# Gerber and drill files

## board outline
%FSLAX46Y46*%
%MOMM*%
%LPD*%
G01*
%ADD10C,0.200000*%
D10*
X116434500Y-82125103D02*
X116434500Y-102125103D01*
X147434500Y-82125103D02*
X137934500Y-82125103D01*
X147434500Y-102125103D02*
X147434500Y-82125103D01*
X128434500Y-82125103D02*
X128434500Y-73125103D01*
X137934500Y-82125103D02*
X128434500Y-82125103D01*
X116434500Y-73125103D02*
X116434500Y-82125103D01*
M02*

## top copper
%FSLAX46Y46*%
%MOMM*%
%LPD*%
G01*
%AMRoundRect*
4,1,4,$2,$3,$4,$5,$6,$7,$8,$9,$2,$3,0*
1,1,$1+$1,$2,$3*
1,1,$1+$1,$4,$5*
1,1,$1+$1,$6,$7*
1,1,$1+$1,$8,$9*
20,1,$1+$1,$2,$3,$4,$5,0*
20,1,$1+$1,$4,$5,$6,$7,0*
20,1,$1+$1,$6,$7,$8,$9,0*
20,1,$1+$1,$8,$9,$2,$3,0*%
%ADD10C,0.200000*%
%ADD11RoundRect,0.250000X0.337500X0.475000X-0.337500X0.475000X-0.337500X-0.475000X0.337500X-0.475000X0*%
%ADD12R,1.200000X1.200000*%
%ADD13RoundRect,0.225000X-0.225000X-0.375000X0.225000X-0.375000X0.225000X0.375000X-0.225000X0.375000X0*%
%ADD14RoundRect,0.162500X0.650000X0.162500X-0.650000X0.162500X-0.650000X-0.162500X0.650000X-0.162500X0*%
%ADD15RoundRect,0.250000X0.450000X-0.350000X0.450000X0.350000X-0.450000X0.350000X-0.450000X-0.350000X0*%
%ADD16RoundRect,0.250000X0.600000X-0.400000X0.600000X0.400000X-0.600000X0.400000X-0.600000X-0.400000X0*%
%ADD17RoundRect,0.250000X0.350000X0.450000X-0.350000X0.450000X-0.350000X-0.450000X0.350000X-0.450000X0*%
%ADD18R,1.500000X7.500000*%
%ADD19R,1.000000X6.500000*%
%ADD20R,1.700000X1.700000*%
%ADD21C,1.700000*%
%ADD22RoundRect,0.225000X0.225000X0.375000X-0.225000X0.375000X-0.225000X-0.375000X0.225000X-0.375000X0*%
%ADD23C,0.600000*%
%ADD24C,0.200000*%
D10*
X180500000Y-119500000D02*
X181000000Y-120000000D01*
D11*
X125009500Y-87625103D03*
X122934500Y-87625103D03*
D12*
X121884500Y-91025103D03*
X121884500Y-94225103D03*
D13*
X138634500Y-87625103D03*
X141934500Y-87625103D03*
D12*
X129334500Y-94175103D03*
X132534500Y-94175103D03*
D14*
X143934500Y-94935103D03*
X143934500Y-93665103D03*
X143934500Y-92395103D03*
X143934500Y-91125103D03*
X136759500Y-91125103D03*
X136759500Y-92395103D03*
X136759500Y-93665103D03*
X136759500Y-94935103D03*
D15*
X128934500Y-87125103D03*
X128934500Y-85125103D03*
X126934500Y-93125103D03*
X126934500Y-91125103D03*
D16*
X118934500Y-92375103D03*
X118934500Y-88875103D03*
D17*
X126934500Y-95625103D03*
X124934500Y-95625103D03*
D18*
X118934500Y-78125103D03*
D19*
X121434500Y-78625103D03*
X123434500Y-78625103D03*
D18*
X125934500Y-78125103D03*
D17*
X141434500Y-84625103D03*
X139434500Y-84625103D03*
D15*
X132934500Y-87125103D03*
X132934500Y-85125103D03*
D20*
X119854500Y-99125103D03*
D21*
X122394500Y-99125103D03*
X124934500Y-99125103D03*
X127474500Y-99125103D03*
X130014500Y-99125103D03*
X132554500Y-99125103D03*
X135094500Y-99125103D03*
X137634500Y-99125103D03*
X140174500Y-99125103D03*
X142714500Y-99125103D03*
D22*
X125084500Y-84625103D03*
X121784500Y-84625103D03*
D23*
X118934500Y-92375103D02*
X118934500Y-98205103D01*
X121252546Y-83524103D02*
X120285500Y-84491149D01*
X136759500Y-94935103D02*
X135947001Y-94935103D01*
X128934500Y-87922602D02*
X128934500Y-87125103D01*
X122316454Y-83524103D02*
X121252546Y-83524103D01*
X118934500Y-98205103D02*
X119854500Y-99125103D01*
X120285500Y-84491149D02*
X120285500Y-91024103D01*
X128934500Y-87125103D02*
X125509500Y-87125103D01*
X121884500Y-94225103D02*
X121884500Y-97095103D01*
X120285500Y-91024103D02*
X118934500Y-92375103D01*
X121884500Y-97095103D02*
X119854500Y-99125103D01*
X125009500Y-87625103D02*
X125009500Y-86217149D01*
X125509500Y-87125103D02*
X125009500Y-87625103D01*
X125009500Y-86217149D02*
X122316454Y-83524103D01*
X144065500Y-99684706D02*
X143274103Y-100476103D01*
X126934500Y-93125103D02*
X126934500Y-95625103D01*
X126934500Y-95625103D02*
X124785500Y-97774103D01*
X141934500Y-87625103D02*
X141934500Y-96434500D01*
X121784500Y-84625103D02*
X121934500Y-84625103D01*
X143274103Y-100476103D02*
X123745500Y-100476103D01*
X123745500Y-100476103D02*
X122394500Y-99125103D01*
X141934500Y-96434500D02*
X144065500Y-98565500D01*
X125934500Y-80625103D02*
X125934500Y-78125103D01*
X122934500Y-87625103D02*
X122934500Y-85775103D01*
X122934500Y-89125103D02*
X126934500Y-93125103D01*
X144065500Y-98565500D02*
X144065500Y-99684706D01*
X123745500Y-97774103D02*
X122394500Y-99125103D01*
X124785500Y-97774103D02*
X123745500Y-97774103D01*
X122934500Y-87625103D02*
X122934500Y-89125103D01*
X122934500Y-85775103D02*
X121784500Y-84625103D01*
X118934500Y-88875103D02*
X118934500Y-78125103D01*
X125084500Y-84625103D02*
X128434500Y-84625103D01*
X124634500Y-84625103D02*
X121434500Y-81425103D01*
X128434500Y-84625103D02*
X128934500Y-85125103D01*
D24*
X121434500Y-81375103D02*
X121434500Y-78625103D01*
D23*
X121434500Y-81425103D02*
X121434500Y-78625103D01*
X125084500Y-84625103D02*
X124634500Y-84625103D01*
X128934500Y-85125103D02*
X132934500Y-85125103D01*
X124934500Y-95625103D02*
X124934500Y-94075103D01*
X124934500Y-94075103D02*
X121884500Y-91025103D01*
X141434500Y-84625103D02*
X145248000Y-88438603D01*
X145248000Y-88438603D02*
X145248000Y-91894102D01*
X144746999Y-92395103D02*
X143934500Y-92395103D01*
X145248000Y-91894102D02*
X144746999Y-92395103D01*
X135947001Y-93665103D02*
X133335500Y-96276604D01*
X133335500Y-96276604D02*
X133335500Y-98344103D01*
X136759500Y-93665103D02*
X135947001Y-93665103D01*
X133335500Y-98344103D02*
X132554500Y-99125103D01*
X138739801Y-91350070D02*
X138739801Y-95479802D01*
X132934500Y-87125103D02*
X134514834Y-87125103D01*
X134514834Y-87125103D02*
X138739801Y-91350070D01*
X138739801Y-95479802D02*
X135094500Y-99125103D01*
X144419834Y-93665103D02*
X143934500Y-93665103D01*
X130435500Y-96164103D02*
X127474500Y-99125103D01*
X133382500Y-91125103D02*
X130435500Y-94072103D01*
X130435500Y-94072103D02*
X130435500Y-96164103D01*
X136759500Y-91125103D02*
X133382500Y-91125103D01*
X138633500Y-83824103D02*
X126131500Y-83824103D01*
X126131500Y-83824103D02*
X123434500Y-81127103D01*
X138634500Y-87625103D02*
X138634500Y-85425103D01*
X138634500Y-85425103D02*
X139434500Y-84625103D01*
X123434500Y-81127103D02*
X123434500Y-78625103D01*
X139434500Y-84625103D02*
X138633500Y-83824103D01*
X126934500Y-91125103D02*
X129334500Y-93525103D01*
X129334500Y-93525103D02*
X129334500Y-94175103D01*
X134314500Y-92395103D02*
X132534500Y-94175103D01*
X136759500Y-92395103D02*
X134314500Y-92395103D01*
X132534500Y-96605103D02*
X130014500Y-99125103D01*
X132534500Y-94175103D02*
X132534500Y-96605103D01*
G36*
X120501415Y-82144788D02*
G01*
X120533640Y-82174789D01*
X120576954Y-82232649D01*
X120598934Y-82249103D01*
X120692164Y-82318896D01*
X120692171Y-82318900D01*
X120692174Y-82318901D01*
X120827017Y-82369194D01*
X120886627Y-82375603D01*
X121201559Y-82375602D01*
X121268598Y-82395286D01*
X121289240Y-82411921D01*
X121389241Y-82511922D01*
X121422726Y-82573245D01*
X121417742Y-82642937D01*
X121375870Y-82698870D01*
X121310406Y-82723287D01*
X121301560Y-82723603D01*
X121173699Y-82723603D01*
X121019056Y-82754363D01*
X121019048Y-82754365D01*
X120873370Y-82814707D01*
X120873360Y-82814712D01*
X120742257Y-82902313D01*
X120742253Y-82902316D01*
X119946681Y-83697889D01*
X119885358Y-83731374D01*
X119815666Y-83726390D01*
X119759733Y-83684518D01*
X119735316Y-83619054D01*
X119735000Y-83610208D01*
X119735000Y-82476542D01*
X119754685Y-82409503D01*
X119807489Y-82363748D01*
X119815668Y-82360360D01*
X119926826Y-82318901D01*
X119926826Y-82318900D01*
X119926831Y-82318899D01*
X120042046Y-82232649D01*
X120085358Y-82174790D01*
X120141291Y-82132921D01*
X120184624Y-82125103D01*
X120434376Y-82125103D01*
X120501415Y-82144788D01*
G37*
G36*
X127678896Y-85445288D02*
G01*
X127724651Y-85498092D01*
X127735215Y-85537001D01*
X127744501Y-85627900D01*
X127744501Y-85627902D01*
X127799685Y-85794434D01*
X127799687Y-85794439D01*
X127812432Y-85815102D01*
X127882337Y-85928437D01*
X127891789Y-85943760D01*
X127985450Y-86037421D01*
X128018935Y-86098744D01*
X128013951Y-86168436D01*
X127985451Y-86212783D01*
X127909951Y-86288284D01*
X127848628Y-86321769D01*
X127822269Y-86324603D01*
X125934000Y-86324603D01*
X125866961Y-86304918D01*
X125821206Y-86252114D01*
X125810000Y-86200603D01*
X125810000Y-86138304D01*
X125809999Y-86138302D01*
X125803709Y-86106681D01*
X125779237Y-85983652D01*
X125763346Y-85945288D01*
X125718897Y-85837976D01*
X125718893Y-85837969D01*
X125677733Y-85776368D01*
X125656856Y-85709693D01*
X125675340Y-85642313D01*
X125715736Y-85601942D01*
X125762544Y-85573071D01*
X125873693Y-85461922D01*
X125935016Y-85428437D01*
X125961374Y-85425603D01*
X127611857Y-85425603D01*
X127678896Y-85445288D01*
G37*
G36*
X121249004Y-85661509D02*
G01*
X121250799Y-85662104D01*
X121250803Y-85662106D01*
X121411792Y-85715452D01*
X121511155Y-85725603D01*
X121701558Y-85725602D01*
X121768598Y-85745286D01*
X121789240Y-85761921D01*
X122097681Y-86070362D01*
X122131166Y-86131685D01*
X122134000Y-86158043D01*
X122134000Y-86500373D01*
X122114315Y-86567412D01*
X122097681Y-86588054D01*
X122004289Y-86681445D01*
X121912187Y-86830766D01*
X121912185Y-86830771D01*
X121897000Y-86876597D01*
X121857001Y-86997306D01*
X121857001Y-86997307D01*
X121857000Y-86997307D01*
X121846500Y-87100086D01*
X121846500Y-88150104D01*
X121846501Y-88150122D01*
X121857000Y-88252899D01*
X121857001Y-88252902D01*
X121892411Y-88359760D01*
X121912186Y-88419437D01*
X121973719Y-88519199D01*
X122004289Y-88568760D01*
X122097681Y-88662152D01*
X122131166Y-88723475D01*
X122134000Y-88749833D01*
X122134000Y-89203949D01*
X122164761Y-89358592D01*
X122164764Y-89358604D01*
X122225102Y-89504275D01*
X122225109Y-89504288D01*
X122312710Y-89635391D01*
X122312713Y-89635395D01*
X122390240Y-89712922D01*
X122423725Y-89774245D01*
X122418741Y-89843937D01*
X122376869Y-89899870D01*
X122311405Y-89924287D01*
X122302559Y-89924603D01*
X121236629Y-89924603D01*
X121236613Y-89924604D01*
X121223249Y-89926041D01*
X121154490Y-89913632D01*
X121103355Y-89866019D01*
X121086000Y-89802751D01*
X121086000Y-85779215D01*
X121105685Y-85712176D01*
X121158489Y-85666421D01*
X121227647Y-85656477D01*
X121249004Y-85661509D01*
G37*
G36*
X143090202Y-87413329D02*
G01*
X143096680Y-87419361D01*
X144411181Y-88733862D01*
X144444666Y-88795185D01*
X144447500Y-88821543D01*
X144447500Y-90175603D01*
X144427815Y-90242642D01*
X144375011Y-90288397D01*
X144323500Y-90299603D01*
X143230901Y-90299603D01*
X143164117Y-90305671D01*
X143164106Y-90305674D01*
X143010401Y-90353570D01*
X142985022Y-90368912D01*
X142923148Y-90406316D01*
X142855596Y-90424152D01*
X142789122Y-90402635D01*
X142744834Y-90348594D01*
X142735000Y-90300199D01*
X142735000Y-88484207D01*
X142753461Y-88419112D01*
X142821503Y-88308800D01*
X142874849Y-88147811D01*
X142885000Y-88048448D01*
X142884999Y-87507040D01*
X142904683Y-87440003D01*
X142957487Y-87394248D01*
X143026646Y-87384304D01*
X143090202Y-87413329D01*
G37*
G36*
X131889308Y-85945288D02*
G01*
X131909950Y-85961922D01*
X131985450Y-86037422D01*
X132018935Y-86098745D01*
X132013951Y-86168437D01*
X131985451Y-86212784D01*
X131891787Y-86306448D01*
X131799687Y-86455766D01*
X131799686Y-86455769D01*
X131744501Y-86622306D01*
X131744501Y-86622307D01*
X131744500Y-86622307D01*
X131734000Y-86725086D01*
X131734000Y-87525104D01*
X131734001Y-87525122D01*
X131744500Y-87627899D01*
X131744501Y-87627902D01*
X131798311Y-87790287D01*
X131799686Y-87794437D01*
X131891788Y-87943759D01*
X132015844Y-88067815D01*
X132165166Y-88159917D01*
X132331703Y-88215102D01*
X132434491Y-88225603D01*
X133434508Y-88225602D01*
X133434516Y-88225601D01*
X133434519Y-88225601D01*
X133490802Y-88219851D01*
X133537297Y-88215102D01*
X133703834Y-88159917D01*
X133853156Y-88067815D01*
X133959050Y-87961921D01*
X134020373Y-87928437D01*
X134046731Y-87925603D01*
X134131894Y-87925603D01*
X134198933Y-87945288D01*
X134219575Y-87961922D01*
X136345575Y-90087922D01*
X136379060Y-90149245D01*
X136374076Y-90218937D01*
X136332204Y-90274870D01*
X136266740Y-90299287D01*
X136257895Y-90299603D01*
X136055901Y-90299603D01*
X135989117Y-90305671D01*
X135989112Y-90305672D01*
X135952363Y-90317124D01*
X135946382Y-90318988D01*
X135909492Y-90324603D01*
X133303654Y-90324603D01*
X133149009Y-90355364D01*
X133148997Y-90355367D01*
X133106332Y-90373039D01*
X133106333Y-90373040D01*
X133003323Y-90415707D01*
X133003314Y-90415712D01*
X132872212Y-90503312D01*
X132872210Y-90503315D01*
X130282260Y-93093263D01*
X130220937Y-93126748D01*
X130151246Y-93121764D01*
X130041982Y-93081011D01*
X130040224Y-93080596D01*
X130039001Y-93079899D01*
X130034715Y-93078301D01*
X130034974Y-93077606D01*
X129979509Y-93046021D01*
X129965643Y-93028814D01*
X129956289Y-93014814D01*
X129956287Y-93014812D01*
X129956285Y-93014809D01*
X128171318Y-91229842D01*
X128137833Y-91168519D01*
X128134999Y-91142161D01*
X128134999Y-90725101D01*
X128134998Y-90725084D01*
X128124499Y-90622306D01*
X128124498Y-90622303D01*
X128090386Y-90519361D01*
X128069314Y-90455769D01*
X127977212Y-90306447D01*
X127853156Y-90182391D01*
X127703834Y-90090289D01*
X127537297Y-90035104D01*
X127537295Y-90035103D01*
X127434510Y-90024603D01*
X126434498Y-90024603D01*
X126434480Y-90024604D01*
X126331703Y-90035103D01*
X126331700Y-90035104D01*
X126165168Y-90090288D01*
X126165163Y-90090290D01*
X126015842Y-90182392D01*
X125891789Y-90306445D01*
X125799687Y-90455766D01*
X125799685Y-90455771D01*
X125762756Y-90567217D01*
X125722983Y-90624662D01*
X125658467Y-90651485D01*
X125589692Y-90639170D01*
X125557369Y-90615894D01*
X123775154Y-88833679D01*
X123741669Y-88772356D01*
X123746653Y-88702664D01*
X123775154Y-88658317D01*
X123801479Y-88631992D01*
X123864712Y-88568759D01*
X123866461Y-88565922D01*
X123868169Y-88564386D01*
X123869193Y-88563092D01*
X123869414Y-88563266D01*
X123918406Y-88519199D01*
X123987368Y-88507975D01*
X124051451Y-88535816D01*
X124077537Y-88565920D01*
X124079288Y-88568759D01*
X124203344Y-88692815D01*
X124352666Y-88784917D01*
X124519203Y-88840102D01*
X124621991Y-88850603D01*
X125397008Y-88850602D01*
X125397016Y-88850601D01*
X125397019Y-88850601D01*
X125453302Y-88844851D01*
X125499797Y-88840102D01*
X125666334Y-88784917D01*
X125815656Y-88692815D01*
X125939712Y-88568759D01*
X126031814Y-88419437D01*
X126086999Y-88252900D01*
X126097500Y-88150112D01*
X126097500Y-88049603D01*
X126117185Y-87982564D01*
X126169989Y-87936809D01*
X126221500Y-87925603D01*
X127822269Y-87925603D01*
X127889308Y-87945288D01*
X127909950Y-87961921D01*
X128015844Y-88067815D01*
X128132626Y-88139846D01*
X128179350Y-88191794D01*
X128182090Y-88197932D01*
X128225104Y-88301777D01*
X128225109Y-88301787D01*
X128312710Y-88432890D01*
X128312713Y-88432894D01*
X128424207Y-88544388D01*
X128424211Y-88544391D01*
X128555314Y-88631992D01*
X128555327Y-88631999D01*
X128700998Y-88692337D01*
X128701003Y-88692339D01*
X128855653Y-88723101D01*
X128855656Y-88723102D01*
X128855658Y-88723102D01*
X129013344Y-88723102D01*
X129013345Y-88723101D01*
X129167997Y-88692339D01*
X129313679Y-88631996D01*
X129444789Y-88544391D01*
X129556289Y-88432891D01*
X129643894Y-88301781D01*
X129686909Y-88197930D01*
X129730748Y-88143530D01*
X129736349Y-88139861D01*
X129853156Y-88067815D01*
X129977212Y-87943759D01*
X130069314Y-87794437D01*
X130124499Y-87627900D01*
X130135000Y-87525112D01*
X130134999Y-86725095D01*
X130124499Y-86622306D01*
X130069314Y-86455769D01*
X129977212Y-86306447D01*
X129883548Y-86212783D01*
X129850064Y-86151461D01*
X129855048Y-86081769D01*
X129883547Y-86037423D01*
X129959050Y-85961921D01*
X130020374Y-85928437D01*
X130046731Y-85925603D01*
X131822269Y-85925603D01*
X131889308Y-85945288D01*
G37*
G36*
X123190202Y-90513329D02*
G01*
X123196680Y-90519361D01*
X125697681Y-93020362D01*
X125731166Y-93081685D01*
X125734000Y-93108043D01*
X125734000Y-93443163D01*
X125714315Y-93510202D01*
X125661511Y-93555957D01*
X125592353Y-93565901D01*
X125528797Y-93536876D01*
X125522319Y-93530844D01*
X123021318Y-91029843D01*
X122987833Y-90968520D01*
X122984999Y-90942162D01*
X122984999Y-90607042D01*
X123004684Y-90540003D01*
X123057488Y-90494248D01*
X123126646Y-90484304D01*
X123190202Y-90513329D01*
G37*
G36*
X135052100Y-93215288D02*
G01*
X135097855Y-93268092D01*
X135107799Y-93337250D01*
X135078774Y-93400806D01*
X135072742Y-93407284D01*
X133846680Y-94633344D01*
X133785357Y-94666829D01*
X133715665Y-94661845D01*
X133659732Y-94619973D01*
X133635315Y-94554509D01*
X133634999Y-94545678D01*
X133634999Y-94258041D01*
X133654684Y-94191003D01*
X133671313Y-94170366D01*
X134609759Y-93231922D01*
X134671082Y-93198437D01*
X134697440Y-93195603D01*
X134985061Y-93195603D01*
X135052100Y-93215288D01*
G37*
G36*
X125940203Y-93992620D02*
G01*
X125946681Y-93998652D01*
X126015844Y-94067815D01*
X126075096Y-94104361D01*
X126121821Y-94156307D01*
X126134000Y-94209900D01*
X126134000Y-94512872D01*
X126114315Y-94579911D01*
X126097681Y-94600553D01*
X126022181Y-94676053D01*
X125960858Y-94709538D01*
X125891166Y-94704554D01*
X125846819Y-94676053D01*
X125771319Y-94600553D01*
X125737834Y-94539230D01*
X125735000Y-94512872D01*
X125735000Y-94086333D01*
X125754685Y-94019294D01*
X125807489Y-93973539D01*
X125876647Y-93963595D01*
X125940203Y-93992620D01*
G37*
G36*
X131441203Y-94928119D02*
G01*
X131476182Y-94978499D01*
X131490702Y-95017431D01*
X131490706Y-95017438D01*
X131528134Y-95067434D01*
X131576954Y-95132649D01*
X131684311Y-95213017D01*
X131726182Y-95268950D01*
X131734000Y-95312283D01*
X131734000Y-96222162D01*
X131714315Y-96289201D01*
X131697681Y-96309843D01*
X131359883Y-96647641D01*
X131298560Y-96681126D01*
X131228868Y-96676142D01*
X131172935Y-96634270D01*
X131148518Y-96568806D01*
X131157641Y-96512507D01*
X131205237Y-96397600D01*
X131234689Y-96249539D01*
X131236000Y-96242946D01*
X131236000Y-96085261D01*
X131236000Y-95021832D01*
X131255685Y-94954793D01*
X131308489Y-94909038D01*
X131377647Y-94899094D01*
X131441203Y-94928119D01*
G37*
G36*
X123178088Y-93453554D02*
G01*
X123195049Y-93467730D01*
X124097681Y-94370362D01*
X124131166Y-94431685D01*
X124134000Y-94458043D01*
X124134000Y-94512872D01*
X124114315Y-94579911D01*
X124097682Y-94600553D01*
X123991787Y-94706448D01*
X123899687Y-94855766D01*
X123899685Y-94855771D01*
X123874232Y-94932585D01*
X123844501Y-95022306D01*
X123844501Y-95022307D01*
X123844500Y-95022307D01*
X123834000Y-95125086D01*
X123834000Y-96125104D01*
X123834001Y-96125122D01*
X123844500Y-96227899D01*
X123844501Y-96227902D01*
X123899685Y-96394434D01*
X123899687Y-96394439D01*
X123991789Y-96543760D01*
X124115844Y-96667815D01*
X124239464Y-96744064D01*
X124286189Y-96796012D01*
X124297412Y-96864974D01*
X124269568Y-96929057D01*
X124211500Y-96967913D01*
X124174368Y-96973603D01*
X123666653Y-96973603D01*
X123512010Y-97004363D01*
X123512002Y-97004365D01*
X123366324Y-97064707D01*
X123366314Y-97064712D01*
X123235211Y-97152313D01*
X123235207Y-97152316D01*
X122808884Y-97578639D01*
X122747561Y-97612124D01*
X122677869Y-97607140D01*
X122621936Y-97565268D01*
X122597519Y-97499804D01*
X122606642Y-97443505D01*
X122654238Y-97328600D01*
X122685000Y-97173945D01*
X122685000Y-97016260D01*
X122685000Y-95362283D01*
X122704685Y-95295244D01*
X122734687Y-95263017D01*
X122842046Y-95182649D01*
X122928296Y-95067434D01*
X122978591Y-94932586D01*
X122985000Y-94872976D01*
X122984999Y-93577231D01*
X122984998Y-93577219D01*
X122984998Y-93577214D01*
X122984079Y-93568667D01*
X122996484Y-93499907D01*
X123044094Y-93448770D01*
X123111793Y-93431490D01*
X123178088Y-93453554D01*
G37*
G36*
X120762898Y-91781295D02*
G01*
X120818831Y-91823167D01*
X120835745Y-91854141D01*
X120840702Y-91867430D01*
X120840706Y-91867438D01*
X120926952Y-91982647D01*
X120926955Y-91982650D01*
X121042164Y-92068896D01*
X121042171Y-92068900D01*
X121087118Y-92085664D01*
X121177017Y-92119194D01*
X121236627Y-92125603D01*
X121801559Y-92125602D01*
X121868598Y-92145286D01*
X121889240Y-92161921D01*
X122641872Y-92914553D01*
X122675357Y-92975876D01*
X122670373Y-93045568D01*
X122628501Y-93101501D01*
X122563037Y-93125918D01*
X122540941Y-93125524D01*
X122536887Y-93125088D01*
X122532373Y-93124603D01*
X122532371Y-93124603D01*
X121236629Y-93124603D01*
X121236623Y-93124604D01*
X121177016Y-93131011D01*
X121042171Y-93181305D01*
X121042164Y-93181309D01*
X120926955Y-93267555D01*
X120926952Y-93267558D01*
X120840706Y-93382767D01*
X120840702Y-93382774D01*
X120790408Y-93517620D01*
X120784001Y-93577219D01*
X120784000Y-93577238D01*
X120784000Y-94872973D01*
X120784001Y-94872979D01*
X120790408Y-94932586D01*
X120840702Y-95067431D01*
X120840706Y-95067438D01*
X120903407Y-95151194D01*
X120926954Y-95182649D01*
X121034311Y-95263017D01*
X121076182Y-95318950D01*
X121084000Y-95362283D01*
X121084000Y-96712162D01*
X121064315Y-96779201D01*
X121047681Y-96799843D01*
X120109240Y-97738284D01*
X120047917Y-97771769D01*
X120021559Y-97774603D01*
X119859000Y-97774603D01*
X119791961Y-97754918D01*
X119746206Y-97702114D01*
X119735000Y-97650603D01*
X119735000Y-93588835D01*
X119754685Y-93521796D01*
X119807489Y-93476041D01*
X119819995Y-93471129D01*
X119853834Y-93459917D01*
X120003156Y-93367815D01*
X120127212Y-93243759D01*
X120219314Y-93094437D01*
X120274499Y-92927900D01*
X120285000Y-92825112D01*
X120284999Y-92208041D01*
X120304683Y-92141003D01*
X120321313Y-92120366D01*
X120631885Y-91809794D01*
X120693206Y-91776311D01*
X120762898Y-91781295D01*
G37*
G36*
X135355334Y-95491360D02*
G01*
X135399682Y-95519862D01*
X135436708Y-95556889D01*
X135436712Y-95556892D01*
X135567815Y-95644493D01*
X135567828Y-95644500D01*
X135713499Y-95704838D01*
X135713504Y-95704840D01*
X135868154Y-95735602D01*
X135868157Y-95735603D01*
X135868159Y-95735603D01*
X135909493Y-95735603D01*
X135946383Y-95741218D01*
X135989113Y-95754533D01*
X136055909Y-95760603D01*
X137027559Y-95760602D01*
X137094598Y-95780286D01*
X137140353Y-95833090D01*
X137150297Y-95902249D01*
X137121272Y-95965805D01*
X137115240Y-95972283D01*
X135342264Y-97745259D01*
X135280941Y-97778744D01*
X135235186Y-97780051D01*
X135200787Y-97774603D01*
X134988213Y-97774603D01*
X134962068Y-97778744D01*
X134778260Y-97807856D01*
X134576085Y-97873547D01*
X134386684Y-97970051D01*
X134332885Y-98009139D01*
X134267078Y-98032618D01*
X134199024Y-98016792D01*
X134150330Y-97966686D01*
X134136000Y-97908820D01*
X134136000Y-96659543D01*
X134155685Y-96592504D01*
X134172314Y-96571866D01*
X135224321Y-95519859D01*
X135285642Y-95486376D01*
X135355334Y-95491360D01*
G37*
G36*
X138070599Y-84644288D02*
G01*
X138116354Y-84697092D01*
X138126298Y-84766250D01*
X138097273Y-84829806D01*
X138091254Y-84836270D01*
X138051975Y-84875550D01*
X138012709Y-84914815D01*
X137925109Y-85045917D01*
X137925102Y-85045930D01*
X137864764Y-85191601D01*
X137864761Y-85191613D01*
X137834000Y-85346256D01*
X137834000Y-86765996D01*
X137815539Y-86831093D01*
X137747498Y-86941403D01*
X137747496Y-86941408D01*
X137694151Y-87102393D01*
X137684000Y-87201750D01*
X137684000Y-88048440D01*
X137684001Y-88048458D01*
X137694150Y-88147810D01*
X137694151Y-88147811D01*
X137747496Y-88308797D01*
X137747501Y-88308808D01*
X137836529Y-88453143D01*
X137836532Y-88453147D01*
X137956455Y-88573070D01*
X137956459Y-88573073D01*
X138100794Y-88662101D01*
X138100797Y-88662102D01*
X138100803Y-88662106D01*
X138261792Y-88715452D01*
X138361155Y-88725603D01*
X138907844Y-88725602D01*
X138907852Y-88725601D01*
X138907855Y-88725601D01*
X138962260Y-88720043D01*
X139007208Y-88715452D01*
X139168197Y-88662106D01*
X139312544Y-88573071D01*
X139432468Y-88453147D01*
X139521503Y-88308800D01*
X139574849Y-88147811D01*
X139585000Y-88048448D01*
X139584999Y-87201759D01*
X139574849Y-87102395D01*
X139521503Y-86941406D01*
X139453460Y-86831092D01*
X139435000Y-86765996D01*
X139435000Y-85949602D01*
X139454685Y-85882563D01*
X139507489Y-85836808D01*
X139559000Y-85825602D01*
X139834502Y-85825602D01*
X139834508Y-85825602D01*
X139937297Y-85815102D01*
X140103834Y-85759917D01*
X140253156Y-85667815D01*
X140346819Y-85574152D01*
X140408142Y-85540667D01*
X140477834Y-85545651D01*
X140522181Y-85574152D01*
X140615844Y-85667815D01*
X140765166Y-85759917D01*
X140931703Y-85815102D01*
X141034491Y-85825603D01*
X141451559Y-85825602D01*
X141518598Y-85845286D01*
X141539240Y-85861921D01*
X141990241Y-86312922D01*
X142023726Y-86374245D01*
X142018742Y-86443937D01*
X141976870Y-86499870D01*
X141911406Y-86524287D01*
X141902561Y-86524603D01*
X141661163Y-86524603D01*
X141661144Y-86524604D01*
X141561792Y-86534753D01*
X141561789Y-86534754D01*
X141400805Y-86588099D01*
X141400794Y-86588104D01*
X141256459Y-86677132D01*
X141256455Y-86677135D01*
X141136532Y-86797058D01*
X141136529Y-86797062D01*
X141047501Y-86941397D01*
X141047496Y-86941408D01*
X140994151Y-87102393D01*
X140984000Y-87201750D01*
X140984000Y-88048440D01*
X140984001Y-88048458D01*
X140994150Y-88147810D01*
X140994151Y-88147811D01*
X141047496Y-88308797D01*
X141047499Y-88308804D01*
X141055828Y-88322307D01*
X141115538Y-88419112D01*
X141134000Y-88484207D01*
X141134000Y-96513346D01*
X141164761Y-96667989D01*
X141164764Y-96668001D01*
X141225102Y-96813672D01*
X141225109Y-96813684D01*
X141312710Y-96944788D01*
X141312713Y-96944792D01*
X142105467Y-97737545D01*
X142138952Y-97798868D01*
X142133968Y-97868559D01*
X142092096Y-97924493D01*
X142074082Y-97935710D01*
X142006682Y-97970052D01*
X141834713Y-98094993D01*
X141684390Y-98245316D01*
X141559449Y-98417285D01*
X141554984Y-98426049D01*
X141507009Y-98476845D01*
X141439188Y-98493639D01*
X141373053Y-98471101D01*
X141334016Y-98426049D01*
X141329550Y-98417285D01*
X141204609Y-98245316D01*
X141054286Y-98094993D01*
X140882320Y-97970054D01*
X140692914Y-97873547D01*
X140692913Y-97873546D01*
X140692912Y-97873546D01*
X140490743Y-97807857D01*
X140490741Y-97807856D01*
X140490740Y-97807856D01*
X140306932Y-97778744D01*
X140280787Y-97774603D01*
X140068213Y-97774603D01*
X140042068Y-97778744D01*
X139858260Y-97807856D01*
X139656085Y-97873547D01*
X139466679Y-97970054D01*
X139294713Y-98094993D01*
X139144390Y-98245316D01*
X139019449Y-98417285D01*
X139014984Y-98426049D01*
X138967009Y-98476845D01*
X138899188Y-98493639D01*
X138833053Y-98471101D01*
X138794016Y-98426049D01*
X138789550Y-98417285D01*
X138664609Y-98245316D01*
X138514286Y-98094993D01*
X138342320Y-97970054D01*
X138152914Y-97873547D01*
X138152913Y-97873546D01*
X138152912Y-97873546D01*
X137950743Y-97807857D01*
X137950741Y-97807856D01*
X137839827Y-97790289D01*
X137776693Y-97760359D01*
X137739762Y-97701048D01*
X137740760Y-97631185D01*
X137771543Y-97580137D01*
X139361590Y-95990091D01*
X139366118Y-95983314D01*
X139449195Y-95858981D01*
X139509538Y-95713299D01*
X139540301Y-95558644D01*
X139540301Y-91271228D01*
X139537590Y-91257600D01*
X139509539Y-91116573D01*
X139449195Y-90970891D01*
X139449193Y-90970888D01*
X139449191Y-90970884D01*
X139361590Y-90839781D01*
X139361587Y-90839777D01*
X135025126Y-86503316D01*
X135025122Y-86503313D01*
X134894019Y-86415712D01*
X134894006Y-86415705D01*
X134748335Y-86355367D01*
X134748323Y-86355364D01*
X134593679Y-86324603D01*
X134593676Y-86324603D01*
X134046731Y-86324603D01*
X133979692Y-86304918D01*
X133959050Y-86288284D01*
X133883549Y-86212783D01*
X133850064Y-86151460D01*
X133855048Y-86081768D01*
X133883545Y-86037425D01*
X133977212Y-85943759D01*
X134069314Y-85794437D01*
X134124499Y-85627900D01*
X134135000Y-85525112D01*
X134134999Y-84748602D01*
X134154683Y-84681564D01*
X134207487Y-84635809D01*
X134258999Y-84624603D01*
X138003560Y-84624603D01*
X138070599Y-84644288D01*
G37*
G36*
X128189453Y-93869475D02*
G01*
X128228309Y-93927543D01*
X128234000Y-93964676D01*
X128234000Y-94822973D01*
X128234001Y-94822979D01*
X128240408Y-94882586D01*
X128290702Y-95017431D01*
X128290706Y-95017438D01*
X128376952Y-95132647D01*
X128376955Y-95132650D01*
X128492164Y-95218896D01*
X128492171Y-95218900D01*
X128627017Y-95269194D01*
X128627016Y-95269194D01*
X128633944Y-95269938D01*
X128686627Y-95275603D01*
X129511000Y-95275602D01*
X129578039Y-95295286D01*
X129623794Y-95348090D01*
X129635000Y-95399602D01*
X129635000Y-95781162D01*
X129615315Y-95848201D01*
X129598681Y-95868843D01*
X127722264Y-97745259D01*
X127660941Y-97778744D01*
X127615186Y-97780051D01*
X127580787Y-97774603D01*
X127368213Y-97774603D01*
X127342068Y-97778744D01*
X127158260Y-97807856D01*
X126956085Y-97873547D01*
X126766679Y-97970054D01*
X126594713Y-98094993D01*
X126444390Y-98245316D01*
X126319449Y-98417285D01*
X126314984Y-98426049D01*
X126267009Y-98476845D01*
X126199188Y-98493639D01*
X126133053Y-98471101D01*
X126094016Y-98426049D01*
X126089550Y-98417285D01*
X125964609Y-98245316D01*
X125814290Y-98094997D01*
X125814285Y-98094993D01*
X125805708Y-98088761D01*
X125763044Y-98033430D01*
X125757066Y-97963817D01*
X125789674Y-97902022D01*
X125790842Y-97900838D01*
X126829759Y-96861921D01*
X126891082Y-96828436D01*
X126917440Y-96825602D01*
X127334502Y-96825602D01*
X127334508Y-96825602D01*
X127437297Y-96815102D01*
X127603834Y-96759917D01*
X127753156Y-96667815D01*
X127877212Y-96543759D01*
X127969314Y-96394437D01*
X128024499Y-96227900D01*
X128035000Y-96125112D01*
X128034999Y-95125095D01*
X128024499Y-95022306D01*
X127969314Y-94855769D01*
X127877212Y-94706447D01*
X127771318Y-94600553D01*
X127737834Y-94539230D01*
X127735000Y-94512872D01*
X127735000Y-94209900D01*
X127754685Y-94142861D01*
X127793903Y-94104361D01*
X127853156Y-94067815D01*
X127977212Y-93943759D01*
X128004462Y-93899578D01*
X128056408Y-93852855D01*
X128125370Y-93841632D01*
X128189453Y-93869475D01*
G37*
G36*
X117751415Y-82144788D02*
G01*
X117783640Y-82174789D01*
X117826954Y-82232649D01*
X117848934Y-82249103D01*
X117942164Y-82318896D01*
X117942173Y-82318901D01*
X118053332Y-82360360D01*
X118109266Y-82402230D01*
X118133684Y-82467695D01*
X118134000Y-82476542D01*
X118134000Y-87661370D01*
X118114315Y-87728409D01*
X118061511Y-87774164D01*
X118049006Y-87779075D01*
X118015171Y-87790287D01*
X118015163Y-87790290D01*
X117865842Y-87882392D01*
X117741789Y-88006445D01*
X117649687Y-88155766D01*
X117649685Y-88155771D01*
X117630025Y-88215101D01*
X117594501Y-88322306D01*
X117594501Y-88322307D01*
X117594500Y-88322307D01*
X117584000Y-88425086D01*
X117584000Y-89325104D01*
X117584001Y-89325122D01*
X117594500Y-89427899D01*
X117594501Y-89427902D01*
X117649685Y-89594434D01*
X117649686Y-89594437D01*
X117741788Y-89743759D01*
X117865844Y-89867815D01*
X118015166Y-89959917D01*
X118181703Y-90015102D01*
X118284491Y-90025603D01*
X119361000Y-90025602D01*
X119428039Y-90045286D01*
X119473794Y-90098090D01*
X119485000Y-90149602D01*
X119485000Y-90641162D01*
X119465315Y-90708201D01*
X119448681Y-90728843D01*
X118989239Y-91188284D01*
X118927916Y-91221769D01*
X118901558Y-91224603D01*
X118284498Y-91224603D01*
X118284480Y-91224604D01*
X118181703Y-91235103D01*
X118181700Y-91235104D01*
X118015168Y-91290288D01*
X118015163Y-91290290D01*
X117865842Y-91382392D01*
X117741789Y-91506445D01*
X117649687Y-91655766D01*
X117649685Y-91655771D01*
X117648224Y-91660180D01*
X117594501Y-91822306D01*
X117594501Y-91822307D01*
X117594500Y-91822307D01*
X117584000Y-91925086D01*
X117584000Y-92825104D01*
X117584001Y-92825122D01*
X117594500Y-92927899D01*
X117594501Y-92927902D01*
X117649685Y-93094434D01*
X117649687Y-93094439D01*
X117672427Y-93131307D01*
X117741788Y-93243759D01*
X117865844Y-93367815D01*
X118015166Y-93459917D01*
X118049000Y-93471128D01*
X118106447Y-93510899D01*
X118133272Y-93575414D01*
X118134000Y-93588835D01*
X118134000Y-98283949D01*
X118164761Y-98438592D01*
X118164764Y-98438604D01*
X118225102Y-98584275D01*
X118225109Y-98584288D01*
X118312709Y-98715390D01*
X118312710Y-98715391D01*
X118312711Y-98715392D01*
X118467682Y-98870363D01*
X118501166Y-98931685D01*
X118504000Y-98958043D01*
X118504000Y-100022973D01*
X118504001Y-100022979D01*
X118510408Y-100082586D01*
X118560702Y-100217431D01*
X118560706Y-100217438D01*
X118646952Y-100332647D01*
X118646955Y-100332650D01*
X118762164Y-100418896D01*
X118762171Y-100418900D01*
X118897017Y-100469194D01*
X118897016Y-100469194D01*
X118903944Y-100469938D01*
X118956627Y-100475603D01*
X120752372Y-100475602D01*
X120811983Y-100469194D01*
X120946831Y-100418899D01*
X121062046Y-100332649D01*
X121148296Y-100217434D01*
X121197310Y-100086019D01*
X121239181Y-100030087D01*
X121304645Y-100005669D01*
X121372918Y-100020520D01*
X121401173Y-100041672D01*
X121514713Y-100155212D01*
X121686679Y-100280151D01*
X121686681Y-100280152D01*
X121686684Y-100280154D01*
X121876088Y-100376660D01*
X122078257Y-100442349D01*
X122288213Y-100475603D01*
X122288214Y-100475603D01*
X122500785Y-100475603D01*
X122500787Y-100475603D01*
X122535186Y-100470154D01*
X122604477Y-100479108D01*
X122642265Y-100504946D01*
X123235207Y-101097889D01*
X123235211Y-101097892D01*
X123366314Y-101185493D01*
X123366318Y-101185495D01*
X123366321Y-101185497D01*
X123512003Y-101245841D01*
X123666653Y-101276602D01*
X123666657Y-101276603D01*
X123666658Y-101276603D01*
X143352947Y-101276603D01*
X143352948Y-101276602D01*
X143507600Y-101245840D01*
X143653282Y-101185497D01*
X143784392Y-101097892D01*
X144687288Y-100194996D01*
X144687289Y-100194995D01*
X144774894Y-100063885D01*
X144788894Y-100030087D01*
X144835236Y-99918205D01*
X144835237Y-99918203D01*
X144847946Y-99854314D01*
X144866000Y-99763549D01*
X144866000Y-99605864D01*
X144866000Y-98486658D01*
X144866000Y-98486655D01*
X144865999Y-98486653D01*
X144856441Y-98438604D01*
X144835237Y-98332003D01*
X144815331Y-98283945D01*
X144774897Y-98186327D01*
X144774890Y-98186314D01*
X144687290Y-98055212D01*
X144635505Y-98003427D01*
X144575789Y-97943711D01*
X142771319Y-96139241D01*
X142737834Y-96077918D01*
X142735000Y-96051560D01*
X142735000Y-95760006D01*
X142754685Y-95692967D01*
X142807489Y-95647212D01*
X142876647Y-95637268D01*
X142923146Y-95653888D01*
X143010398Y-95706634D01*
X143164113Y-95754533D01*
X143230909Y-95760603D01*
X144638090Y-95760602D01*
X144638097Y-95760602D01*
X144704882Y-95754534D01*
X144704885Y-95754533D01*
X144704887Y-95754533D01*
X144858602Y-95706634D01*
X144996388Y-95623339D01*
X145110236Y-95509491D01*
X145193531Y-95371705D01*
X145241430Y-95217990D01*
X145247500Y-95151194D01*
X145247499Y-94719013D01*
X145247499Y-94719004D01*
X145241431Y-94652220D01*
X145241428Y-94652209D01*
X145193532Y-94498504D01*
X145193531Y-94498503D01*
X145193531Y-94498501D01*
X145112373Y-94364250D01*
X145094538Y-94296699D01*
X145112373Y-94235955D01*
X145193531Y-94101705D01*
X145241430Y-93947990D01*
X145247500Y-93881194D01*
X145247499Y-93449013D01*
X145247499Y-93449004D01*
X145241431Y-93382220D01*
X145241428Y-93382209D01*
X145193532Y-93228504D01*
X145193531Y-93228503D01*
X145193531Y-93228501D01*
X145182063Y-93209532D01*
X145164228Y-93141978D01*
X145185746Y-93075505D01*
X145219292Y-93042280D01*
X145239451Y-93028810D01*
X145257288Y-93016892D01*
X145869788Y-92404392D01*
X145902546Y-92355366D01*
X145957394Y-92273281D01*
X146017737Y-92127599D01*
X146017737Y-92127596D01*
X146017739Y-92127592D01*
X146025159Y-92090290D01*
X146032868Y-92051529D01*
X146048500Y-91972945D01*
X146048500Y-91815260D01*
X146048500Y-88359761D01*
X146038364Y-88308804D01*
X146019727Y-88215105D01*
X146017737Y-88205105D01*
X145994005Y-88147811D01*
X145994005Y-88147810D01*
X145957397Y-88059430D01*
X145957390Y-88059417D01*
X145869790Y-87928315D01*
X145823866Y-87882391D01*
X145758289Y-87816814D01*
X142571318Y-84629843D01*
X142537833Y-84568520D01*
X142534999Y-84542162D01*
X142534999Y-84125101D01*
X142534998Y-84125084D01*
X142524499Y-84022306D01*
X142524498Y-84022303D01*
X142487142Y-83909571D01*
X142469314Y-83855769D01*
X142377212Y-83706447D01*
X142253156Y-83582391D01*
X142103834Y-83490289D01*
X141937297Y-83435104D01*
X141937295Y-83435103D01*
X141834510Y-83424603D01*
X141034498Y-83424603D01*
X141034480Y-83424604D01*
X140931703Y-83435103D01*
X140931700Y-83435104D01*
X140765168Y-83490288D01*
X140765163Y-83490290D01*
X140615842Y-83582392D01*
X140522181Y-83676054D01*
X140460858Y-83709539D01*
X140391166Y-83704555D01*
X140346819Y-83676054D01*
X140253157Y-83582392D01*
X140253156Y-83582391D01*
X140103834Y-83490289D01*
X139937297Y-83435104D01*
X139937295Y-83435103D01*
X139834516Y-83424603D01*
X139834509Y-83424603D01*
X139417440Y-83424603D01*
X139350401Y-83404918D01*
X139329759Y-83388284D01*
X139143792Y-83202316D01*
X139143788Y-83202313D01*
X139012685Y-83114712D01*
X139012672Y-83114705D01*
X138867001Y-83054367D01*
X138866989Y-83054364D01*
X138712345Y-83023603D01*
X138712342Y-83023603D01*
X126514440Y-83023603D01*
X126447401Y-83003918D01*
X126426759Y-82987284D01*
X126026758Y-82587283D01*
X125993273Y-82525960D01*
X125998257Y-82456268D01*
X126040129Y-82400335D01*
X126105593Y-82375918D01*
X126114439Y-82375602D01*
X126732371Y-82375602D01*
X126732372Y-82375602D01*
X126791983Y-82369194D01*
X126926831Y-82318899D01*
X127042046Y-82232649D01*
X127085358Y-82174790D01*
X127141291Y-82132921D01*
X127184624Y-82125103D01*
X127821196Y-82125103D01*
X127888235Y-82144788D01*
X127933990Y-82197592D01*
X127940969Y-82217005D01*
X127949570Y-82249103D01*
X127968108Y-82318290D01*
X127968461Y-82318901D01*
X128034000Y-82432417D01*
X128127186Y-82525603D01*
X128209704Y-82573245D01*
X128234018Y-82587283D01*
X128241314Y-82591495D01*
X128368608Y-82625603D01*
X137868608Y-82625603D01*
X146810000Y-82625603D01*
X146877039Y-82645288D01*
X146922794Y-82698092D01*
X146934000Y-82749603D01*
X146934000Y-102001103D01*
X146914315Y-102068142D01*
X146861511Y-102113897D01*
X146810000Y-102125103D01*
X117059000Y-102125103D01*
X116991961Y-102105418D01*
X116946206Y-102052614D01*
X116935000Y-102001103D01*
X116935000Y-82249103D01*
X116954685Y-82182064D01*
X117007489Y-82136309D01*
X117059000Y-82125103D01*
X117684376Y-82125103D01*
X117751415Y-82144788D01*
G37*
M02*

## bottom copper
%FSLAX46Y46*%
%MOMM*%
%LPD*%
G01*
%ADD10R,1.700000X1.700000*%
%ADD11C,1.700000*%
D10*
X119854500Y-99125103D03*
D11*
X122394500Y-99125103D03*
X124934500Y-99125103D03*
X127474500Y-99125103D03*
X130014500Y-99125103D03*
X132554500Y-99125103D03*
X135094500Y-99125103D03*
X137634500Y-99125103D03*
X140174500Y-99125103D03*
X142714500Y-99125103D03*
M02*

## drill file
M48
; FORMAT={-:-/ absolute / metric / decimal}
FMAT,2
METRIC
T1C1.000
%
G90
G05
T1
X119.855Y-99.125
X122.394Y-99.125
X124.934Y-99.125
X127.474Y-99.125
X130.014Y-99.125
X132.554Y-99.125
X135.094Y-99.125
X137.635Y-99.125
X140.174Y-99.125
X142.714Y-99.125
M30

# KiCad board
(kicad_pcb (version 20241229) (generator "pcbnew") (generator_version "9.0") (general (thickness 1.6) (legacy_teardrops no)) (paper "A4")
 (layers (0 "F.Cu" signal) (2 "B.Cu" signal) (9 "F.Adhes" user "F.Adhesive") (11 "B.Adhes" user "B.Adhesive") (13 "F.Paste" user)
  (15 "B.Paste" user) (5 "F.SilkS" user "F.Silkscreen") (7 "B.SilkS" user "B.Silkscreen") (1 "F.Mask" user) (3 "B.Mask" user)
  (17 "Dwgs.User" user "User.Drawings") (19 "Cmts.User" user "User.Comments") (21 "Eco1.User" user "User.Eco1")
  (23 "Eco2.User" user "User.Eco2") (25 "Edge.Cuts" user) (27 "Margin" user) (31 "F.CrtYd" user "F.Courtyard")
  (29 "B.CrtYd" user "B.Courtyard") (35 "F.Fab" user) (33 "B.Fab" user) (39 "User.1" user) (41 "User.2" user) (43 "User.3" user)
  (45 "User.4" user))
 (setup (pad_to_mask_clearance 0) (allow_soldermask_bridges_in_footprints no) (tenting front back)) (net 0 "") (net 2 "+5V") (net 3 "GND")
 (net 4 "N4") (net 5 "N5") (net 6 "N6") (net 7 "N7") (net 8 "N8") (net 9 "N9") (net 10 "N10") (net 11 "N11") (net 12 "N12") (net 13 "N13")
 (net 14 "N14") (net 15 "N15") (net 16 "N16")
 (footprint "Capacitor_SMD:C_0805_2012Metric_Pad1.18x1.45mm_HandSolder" (layer "F.Cu") (at 123.972 87.625103 180)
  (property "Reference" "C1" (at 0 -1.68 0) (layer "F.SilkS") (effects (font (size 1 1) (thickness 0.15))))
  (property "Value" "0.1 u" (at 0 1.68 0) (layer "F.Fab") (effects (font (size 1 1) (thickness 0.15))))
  (pad "1" smd roundrect (at -1.0375 0 180) (size 1.175 1.45) (layers "F.Cu" "F.Mask" "F.Paste") (roundrect_rratio 0.212766) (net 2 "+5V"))
  (pad "2" smd roundrect (at 1.0375 0 180) (size 1.175 1.45) (layers "F.Cu" "F.Mask" "F.Paste") (roundrect_rratio 0.212766) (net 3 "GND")))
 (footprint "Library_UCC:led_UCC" (layer "F.Cu") (at 122.3345 93.125103 -90)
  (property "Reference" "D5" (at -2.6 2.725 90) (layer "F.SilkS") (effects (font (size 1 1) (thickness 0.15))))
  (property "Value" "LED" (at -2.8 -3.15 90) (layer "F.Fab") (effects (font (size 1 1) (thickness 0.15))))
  (pad "1" smd rect (at -2.1 0.45 270) (size 1.2 1.2) (layers "F.Cu" "F.Mask" "F.Paste") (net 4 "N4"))
  (pad "2" smd rect (at 1.1 0.45 270) (size 1.2 1.2) (layers "F.Cu" "F.Mask" "F.Paste") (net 2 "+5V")))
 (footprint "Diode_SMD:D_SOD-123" (layer "F.Cu") (at 140.2845 87.625103)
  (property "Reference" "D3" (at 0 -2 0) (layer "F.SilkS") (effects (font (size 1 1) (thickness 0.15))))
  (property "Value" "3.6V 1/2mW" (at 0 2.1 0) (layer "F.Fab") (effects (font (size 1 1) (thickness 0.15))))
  (pad "1" smd roundrect (at -1.65 0) (size 0.9 1.2) (layers "F.Cu" "F.Mask" "F.Paste") (roundrect_rratio 0.25) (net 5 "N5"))
  (pad "2" smd roundrect (at 1.65 0) (size 0.9 1.2) (layers "F.Cu" "F.Mask" "F.Paste") (roundrect_rratio 0.25) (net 3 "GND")))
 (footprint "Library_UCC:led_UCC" (layer "F.Cu") (at 131.4345 93.725103)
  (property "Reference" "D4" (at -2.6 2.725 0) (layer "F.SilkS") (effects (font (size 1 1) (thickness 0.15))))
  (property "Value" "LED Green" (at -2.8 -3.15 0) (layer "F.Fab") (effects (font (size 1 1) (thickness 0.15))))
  (pad "1" smd rect (at -2.1 0.45) (size 1.2 1.2) (layers "F.Cu" "F.Mask" "F.Paste") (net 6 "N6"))
  (pad "2" smd rect (at 1.1 0.45) (size 1.2 1.2) (layers "F.Cu" "F.Mask" "F.Paste") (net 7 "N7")))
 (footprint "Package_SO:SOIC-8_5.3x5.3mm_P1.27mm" (layer "F.Cu") (at 140.347 93.030103 180)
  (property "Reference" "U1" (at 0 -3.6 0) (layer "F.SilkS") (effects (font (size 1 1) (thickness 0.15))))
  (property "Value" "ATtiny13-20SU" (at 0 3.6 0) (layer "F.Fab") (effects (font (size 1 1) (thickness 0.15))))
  (pad "1" smd roundrect (at -3.5875 -1.905 180) (size 1.625 0.65) (layers "F.Cu" "F.Mask" "F.Paste") (roundrect_rratio 0.25) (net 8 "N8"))
  (pad "2" smd roundrect (at -3.5875 -0.635 180) (size 1.625 0.65) (layers "F.Cu" "F.Mask" "F.Paste") (roundrect_rratio 0.25) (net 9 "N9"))
  (pad "3" smd roundrect (at -3.5875 0.635 180) (size 1.625 0.65) (layers "F.Cu" "F.Mask" "F.Paste") (roundrect_rratio 0.25) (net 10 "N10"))
  (pad "4" smd roundrect (at -3.5875 1.905 180) (size 1.625 0.65) (layers "F.Cu" "F.Mask" "F.Paste") (roundrect_rratio 0.25) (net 3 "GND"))
  (pad "5" smd roundrect (at 3.5875 1.905 180) (size 1.625 0.65) (layers "F.Cu" "F.Mask" "F.Paste") (roundrect_rratio 0.25) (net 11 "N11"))
  (pad "6" smd roundrect (at 3.5875 0.635 180) (size 1.625 0.65) (layers "F.Cu" "F.Mask" "F.Paste") (roundrect_rratio 0.25) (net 7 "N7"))
  (pad "7" smd roundrect (at 3.5875 -0.635 180) (size 1.625 0.65) (layers "F.Cu" "F.Mask" "F.Paste") (roundrect_rratio 0.25) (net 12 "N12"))
  (pad "8" smd roundrect (at 3.5875 -1.905 180) (size 1.625 0.65) (layers "F.Cu" "F.Mask" "F.Paste") (roundrect_rratio 0.25) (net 2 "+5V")))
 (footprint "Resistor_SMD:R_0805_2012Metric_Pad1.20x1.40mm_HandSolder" (layer "F.Cu") (at 128.9345 86.125103 90)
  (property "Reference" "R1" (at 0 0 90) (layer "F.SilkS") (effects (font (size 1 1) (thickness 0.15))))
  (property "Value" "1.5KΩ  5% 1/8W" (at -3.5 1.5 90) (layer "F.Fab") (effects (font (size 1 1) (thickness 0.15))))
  (pad "1" smd roundrect (at -1 0 90) (size 1.2 1.4) (layers "F.Cu" "F.Mask" "F.Paste") (roundrect_rratio 0.208333) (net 2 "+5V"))
  (pad "2" smd roundrect (at 1 0 90) (size 1.2 1.4) (layers "F.Cu" "F.Mask" "F.Paste") (roundrect_rratio 0.208333) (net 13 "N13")))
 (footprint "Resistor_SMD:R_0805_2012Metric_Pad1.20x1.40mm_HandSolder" (layer "F.Cu") (at 126.9345 92.125103 90)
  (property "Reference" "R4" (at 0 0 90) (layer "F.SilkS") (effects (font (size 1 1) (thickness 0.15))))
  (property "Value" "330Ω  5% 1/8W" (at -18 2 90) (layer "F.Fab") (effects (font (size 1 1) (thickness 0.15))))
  (pad "1" smd roundrect (at -1 0 90) (size 1.2 1.4) (layers "F.Cu" "F.Mask" "F.Paste") (roundrect_rratio 0.208333) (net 3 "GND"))
  (pad "2" smd roundrect (at 1 0 90) (size 1.2 1.4) (layers "F.Cu" "F.Mask" "F.Paste") (roundrect_rratio 0.208333) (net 6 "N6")))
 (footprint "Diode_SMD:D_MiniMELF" (layer "F.Cu") (at 118.9345 90.625103 90)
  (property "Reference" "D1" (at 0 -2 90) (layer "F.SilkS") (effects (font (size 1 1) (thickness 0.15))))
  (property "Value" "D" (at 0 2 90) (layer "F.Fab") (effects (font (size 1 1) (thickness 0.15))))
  (pad "1" smd roundrect (at -1.75 0 90) (size 1.3 1.7) (layers "F.Cu" "F.Mask" "F.Paste") (roundrect_rratio 0.1923076923) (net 2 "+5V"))
  (pad "2" smd roundrect (at 1.75 0 90) (size 1.3 1.7) (layers "F.Cu" "F.Mask" "F.Paste") (roundrect_rratio 0.1923076923) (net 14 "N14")))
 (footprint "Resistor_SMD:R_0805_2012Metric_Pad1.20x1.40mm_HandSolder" (layer "F.Cu") (at 125.9345 95.625103 180)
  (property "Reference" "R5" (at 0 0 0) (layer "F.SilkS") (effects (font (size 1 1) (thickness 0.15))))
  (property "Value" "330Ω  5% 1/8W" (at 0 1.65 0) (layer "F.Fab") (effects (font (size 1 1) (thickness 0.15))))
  (pad "1" smd roundrect (at -1 0 180) (size 1.2 1.4) (layers "F.Cu" "F.Mask" "F.Paste") (roundrect_rratio 0.208333) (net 3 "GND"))
  (pad "2" smd roundrect (at 1 0 180) (size 1.2 1.4) (layers "F.Cu" "F.Mask" "F.Paste") (roundrect_rratio 0.208333) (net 4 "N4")))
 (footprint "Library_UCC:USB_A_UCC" (layer "F.Cu") (at 122.4345 78.325103 -90)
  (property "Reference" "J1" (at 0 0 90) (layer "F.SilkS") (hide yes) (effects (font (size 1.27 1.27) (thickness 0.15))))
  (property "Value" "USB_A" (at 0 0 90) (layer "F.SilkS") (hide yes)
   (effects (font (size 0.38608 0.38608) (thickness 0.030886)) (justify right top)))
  (pad "1" smd rect (at -0.2 3.5 270) (size 7.5 1.5) (layers "F.Cu" "F.Mask" "F.Paste") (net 14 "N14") (solder_mask_margin 0.1016))
  (pad "2" smd rect (at 0.3 1 270) (size 6.5 1) (layers "F.Cu" "F.Mask" "F.Paste") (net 13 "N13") (solder_mask_margin 0.1016))
  (pad "3" smd rect (at 0.3 -1 270) (size 6.5 1) (layers "F.Cu" "F.Mask" "F.Paste") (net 5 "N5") (solder_mask_margin 0.1016))
  (pad "4" smd rect (at -0.2 -3.5 270) (size 7.5 1.5) (layers "F.Cu" "F.Mask" "F.Paste") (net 3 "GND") (solder_mask_margin 0.1016)))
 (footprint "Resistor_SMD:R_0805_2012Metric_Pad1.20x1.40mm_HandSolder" (layer "F.Cu") (at 140.4345 84.625103 180)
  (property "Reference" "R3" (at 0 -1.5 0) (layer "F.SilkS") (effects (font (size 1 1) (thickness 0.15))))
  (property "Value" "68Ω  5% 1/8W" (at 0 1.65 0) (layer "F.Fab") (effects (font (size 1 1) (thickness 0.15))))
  (pad "1" smd roundrect (at -1 0 180) (size 1.2 1.4) (layers "F.Cu" "F.Mask" "F.Paste") (roundrect_rratio 0.208333) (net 10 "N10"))
  (pad "2" smd roundrect (at 1 0 180) (size 1.2 1.4) (layers "F.Cu" "F.Mask" "F.Paste") (roundrect_rratio 0.208333) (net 5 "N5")))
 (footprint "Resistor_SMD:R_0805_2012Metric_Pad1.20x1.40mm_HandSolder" (layer "F.Cu") (at 132.9345 86.125103 90)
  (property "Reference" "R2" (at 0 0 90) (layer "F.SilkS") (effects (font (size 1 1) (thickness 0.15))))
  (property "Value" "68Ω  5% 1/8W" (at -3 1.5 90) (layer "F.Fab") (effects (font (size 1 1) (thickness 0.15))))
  (pad "1" smd roundrect (at -1 0 90) (size 1.2 1.4) (layers "F.Cu" "F.Mask" "F.Paste") (roundrect_rratio 0.208333) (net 9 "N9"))
  (pad "2" smd roundrect (at 1 0 90) (size 1.2 1.4) (layers "F.Cu" "F.Mask" "F.Paste") (roundrect_rratio 0.208333) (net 13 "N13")))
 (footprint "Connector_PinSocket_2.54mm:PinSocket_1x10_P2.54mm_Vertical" (layer "F.Cu") (at 119.8545 99.125103 90)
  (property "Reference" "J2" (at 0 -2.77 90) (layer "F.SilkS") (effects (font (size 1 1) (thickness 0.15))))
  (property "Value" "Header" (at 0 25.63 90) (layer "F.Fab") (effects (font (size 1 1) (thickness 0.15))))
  (pad "1" thru_hole rect (at 0 0 90) (size 1.7 1.7) (drill 1) (layers "*.Cu" "*.Mask") (remove_unused_layers no) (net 2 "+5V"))
  (pad "2" thru_hole circle (at 0 2.54 90) (size 1.7 1.7) (drill 1) (layers "*.Cu" "*.Mask") (remove_unused_layers no) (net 3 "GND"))
  (pad "3" thru_hole circle (at 0 5.08 90) (size 1.7 1.7) (drill 1) (layers "*.Cu" "*.Mask") (remove_unused_layers no) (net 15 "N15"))
  (pad "4" thru_hole circle (at 0 7.62 90) (size 1.7 1.7) (drill 1) (layers "*.Cu" "*.Mask") (remove_unused_layers no) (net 11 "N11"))
  (pad "5" thru_hole circle (at 0 10.16 90) (size 1.7 1.7) (drill 1) (layers "*.Cu" "*.Mask") (remove_unused_layers no) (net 7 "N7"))
  (pad "6" thru_hole circle (at 0 12.7 90) (size 1.7 1.7) (drill 1) (layers "*.Cu" "*.Mask") (remove_unused_layers no) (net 12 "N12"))
  (pad "7" thru_hole circle (at 0 15.24 90) (size 1.7 1.7) (drill 1) (layers "*.Cu" "*.Mask") (remove_unused_layers no) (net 9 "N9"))
  (pad "8" thru_hole circle (at 0 17.78 90) (size 1.7 1.7) (drill 1) (layers "*.Cu" "*.Mask") (remove_unused_layers no) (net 10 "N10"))
  (pad "9" thru_hole circle (at 0 20.32 90) (size 1.7 1.7) (drill 1) (layers "*.Cu" "*.Mask") (remove_unused_layers no) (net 8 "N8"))
  (pad "10" thru_hole circle (at 0 22.86 90) (size 1.7 1.7) (drill 1) (layers "*.Cu" "*.Mask") (remove_unused_layers no) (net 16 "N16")))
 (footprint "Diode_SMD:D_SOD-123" (layer "F.Cu") (at 123.4345 84.625103 180)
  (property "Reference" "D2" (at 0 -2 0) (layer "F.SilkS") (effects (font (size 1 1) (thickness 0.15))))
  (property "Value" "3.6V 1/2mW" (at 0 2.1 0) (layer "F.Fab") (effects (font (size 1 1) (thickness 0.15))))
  (pad "1" smd roundrect (at -1.65 0 180) (size 0.9 1.2) (layers "F.Cu" "F.Mask" "F.Paste") (roundrect_rratio 0.25) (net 13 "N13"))
  (pad "2" smd roundrect (at 1.65 0 180) (size 0.9 1.2) (layers "F.Cu" "F.Mask" "F.Paste") (roundrect_rratio 0.25) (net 3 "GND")))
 (gr_line (start 180.5 119.5) (end 181 120) (stroke (width 0.2) (type default)) (layer "F.Cu"))
 (gr_line (start 116.4345 82.125103) (end 116.4345 102.125103) (stroke (width 0.2) (type solid)) (layer "Edge.Cuts"))
 (gr_line (start 147.4345 82.125103) (end 137.9345 82.125103) (stroke (width 0.2) (type solid)) (layer "Edge.Cuts"))
 (gr_line (start 147.4345 102.125103) (end 147.4345 82.125103) (stroke (width 0.2) (type solid)) (layer "Edge.Cuts"))
 (gr_line (start 128.4345 82.125103) (end 128.4345 73.125103) (stroke (width 0.2) (type solid)) (layer "Edge.Cuts"))
 (gr_line (start 137.9345 82.125103) (end 128.4345 82.125103) (stroke (width 0.2) (type solid)) (layer "Edge.Cuts"))
 (gr_line (start 116.4345 73.125103) (end 116.4345 82.125103) (stroke (width 0.2) (type solid)) (layer "Edge.Cuts"))
 (segment (start 118.9345 92.375103) (end 118.9345 98.205103) (width 0.6) (layer "F.Cu") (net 2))
 (segment (start 121.252546 83.524103) (end 120.2855 84.491149) (width 0.6) (layer "F.Cu") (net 2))
 (segment (start 136.7595 94.935103) (end 135.947001 94.935103) (width 0.6) (layer "F.Cu") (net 2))
 (segment (start 128.9345 87.922602) (end 128.9345 87.125103) (width 0.6) (layer "F.Cu") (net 2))
 (segment (start 122.316454 83.524103) (end 121.252546 83.524103) (width 0.6) (layer "F.Cu") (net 2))
 (segment (start 118.9345 98.205103) (end 119.8545 99.125103) (width 0.6) (layer "F.Cu") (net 2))
 (segment (start 120.2855 84.491149) (end 120.2855 91.024103) (width 0.6) (layer "F.Cu") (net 2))
 (segment (start 128.9345 87.125103) (end 125.5095 87.125103) (width 0.6) (layer "F.Cu") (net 2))
 (segment (start 121.8845 94.225103) (end 121.8845 97.095103) (width 0.6) (layer "F.Cu") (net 2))
 (segment (start 120.2855 91.024103) (end 118.9345 92.375103) (width 0.6) (layer "F.Cu") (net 2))
 (segment (start 121.8845 97.095103) (end 119.8545 99.125103) (width 0.6) (layer "F.Cu") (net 2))
 (segment (start 125.0095 87.625103) (end 125.0095 86.217149) (width 0.6) (layer "F.Cu") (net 2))
 (segment (start 125.5095 87.125103) (end 125.0095 87.625103) (width 0.6) (layer "F.Cu") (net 2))
 (segment (start 125.0095 86.217149) (end 122.316454 83.524103) (width 0.6) (layer "F.Cu") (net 2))
 (segment (start 144.0655 99.684706) (end 143.274103 100.476103) (width 0.6) (layer "F.Cu") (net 3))
 (segment (start 126.9345 93.125103) (end 126.9345 95.625103) (width 0.6) (layer "F.Cu") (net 3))
 (segment (start 126.9345 95.625103) (end 124.7855 97.774103) (width 0.6) (layer "F.Cu") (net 3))
 (segment (start 141.9345 87.625103) (end 141.9345 96.4345) (width 0.6) (layer "F.Cu") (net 3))
 (segment (start 121.7845 84.625103) (end 121.9345 84.625103) (width 0.6) (layer "F.Cu") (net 3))
 (segment (start 143.274103 100.476103) (end 123.7455 100.476103) (width 0.6) (layer "F.Cu") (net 3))
 (segment (start 123.7455 100.476103) (end 122.3945 99.125103) (width 0.6) (layer "F.Cu") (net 3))
 (segment (start 141.9345 96.4345) (end 144.0655 98.5655) (width 0.6) (layer "F.Cu") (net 3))
 (segment (start 125.9345 80.625103) (end 125.9345 78.125103) (width 0.6) (layer "F.Cu") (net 3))
 (segment (start 122.9345 87.625103) (end 122.9345 85.775103) (width 0.6) (layer "F.Cu") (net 3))
 (segment (start 122.9345 89.125103) (end 126.9345 93.125103) (width 0.6) (layer "F.Cu") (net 3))
 (segment (start 144.0655 98.5655) (end 144.0655 99.684706) (width 0.6) (layer "F.Cu") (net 3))
 (segment (start 123.7455 97.774103) (end 122.3945 99.125103) (width 0.6) (layer "F.Cu") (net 3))
 (segment (start 124.7855 97.774103) (end 123.7455 97.774103) (width 0.6) (layer "F.Cu") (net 3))
 (segment (start 122.9345 87.625103) (end 122.9345 89.125103) (width 0.6) (layer "F.Cu") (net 3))
 (segment (start 122.9345 85.775103) (end 121.7845 84.625103) (width 0.6) (layer "F.Cu") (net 3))
 (segment (start 118.9345 88.875103) (end 118.9345 78.125103) (width 0.6) (layer "F.Cu") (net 14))
 (segment (start 125.0845 84.625103) (end 128.4345 84.625103) (width 0.6) (layer "F.Cu") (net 13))
 (segment (start 124.6345 84.625103) (end 121.4345 81.425103) (width 0.6) (layer "F.Cu") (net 13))
 (segment (start 128.4345 84.625103) (end 128.9345 85.125103) (width 0.6) (layer "F.Cu") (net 13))
 (segment (start 121.4345 81.375103) (end 121.4345 78.625103) (width 0.2) (layer "F.Cu") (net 13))
 (segment (start 121.4345 81.425103) (end 121.4345 78.625103) (width 0.6) (layer "F.Cu") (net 13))
 (segment (start 125.0845 84.625103) (end 124.6345 84.625103) (width 0.6) (layer "F.Cu") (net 13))
 (segment (start 128.9345 85.125103) (end 132.9345 85.125103) (width 0.6) (layer "F.Cu") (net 13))
 (segment (start 124.9345 95.625103) (end 124.9345 94.075103) (width 0.6) (layer "F.Cu") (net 4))
 (segment (start 124.9345 94.075103) (end 121.8845 91.025103) (width 0.6) (layer "F.Cu") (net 4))
 (segment (start 141.4345 84.625103) (end 145.248 88.438603) (width 0.6) (layer "F.Cu") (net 10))
 (segment (start 145.248 88.438603) (end 145.248 91.894102) (width 0.6) (layer "F.Cu") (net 10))
 (segment (start 144.746999 92.395103) (end 143.9345 92.395103) (width 0.6) (layer "F.Cu") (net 10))
 (segment (start 145.248 91.894102) (end 144.746999 92.395103) (width 0.6) (layer "F.Cu") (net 10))
 (segment (start 135.947001 93.665103) (end 133.3355 96.276604) (width 0.6) (layer "F.Cu") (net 12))
 (segment (start 133.3355 96.276604) (end 133.3355 98.344103) (width 0.6) (layer "F.Cu") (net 12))
 (segment (start 136.7595 93.665103) (end 135.947001 93.665103) (width 0.6) (layer "F.Cu") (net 12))
 (segment (start 133.3355 98.344103) (end 132.5545 99.125103) (width 0.6) (layer "F.Cu") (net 12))
 (segment (start 138.739801 91.35007) (end 138.739801 95.479802) (width 0.6) (layer "F.Cu") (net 9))
 (segment (start 132.9345 87.125103) (end 134.514834 87.125103) (width 0.6) (layer "F.Cu") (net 9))
 (segment (start 134.514834 87.125103) (end 138.739801 91.35007) (width 0.6) (layer "F.Cu") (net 9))
 (segment (start 138.739801 95.479802) (end 135.0945 99.125103) (width 0.6) (layer "F.Cu") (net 9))
 (segment (start 144.419834 93.665103) (end 143.9345 93.665103) (width 0.6) (layer "F.Cu") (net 9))
 (segment (start 130.4355 96.164103) (end 127.4745 99.125103) (width 0.6) (layer "F.Cu") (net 11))
 (segment (start 133.3825 91.125103) (end 130.4355 94.072103) (width 0.6) (layer "F.Cu") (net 11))
 (segment (start 130.4355 94.072103) (end 130.4355 96.164103) (width 0.6) (layer "F.Cu") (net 11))
 (segment (start 136.7595 91.125103) (end 133.3825 91.125103) (width 0.6) (layer "F.Cu") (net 11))
 (segment (start 138.6335 83.824103) (end 126.1315 83.824103) (width 0.6) (layer "F.Cu") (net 5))
 (segment (start 126.1315 83.824103) (end 123.4345 81.127103) (width 0.6) (layer "F.Cu") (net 5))
 (segment (start 138.6345 87.625103) (end 138.6345 85.425103) (width 0.6) (layer "F.Cu") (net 5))
 (segment (start 138.6345 85.425103) (end 139.4345 84.625103) (width 0.6) (layer "F.Cu") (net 5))
 (segment (start 123.4345 81.127103) (end 123.4345 78.625103) (width 0.6) (layer "F.Cu") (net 5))
 (segment (start 139.4345 84.625103) (end 138.6335 83.824103) (width 0.6) (layer "F.Cu") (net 5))
 (segment (start 126.9345 91.125103) (end 129.3345 93.525103) (width 0.6) (layer "F.Cu") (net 6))
 (segment (start 129.3345 93.525103) (end 129.3345 94.175103) (width 0.6) (layer "F.Cu") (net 6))
 (segment (start 134.3145 92.395103) (end 132.5345 94.175103) (width 0.6) (layer "F.Cu") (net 7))
 (segment (start 136.7595 92.395103) (end 134.3145 92.395103) (width 0.6) (layer "F.Cu") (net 7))
 (segment (start 132.5345 96.605103) (end 130.0145 99.125103) (width 0.6) (layer "F.Cu") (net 7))
 (segment (start 132.5345 94.175103) (end 132.5345 96.605103) (width 0.6) (layer "F.Cu") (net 7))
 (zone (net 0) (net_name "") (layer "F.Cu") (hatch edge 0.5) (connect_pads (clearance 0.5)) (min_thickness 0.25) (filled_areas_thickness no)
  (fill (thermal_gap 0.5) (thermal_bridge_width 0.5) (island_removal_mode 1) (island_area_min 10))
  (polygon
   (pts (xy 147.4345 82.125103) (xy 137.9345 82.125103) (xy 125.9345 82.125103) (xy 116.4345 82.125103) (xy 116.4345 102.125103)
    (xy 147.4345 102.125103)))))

